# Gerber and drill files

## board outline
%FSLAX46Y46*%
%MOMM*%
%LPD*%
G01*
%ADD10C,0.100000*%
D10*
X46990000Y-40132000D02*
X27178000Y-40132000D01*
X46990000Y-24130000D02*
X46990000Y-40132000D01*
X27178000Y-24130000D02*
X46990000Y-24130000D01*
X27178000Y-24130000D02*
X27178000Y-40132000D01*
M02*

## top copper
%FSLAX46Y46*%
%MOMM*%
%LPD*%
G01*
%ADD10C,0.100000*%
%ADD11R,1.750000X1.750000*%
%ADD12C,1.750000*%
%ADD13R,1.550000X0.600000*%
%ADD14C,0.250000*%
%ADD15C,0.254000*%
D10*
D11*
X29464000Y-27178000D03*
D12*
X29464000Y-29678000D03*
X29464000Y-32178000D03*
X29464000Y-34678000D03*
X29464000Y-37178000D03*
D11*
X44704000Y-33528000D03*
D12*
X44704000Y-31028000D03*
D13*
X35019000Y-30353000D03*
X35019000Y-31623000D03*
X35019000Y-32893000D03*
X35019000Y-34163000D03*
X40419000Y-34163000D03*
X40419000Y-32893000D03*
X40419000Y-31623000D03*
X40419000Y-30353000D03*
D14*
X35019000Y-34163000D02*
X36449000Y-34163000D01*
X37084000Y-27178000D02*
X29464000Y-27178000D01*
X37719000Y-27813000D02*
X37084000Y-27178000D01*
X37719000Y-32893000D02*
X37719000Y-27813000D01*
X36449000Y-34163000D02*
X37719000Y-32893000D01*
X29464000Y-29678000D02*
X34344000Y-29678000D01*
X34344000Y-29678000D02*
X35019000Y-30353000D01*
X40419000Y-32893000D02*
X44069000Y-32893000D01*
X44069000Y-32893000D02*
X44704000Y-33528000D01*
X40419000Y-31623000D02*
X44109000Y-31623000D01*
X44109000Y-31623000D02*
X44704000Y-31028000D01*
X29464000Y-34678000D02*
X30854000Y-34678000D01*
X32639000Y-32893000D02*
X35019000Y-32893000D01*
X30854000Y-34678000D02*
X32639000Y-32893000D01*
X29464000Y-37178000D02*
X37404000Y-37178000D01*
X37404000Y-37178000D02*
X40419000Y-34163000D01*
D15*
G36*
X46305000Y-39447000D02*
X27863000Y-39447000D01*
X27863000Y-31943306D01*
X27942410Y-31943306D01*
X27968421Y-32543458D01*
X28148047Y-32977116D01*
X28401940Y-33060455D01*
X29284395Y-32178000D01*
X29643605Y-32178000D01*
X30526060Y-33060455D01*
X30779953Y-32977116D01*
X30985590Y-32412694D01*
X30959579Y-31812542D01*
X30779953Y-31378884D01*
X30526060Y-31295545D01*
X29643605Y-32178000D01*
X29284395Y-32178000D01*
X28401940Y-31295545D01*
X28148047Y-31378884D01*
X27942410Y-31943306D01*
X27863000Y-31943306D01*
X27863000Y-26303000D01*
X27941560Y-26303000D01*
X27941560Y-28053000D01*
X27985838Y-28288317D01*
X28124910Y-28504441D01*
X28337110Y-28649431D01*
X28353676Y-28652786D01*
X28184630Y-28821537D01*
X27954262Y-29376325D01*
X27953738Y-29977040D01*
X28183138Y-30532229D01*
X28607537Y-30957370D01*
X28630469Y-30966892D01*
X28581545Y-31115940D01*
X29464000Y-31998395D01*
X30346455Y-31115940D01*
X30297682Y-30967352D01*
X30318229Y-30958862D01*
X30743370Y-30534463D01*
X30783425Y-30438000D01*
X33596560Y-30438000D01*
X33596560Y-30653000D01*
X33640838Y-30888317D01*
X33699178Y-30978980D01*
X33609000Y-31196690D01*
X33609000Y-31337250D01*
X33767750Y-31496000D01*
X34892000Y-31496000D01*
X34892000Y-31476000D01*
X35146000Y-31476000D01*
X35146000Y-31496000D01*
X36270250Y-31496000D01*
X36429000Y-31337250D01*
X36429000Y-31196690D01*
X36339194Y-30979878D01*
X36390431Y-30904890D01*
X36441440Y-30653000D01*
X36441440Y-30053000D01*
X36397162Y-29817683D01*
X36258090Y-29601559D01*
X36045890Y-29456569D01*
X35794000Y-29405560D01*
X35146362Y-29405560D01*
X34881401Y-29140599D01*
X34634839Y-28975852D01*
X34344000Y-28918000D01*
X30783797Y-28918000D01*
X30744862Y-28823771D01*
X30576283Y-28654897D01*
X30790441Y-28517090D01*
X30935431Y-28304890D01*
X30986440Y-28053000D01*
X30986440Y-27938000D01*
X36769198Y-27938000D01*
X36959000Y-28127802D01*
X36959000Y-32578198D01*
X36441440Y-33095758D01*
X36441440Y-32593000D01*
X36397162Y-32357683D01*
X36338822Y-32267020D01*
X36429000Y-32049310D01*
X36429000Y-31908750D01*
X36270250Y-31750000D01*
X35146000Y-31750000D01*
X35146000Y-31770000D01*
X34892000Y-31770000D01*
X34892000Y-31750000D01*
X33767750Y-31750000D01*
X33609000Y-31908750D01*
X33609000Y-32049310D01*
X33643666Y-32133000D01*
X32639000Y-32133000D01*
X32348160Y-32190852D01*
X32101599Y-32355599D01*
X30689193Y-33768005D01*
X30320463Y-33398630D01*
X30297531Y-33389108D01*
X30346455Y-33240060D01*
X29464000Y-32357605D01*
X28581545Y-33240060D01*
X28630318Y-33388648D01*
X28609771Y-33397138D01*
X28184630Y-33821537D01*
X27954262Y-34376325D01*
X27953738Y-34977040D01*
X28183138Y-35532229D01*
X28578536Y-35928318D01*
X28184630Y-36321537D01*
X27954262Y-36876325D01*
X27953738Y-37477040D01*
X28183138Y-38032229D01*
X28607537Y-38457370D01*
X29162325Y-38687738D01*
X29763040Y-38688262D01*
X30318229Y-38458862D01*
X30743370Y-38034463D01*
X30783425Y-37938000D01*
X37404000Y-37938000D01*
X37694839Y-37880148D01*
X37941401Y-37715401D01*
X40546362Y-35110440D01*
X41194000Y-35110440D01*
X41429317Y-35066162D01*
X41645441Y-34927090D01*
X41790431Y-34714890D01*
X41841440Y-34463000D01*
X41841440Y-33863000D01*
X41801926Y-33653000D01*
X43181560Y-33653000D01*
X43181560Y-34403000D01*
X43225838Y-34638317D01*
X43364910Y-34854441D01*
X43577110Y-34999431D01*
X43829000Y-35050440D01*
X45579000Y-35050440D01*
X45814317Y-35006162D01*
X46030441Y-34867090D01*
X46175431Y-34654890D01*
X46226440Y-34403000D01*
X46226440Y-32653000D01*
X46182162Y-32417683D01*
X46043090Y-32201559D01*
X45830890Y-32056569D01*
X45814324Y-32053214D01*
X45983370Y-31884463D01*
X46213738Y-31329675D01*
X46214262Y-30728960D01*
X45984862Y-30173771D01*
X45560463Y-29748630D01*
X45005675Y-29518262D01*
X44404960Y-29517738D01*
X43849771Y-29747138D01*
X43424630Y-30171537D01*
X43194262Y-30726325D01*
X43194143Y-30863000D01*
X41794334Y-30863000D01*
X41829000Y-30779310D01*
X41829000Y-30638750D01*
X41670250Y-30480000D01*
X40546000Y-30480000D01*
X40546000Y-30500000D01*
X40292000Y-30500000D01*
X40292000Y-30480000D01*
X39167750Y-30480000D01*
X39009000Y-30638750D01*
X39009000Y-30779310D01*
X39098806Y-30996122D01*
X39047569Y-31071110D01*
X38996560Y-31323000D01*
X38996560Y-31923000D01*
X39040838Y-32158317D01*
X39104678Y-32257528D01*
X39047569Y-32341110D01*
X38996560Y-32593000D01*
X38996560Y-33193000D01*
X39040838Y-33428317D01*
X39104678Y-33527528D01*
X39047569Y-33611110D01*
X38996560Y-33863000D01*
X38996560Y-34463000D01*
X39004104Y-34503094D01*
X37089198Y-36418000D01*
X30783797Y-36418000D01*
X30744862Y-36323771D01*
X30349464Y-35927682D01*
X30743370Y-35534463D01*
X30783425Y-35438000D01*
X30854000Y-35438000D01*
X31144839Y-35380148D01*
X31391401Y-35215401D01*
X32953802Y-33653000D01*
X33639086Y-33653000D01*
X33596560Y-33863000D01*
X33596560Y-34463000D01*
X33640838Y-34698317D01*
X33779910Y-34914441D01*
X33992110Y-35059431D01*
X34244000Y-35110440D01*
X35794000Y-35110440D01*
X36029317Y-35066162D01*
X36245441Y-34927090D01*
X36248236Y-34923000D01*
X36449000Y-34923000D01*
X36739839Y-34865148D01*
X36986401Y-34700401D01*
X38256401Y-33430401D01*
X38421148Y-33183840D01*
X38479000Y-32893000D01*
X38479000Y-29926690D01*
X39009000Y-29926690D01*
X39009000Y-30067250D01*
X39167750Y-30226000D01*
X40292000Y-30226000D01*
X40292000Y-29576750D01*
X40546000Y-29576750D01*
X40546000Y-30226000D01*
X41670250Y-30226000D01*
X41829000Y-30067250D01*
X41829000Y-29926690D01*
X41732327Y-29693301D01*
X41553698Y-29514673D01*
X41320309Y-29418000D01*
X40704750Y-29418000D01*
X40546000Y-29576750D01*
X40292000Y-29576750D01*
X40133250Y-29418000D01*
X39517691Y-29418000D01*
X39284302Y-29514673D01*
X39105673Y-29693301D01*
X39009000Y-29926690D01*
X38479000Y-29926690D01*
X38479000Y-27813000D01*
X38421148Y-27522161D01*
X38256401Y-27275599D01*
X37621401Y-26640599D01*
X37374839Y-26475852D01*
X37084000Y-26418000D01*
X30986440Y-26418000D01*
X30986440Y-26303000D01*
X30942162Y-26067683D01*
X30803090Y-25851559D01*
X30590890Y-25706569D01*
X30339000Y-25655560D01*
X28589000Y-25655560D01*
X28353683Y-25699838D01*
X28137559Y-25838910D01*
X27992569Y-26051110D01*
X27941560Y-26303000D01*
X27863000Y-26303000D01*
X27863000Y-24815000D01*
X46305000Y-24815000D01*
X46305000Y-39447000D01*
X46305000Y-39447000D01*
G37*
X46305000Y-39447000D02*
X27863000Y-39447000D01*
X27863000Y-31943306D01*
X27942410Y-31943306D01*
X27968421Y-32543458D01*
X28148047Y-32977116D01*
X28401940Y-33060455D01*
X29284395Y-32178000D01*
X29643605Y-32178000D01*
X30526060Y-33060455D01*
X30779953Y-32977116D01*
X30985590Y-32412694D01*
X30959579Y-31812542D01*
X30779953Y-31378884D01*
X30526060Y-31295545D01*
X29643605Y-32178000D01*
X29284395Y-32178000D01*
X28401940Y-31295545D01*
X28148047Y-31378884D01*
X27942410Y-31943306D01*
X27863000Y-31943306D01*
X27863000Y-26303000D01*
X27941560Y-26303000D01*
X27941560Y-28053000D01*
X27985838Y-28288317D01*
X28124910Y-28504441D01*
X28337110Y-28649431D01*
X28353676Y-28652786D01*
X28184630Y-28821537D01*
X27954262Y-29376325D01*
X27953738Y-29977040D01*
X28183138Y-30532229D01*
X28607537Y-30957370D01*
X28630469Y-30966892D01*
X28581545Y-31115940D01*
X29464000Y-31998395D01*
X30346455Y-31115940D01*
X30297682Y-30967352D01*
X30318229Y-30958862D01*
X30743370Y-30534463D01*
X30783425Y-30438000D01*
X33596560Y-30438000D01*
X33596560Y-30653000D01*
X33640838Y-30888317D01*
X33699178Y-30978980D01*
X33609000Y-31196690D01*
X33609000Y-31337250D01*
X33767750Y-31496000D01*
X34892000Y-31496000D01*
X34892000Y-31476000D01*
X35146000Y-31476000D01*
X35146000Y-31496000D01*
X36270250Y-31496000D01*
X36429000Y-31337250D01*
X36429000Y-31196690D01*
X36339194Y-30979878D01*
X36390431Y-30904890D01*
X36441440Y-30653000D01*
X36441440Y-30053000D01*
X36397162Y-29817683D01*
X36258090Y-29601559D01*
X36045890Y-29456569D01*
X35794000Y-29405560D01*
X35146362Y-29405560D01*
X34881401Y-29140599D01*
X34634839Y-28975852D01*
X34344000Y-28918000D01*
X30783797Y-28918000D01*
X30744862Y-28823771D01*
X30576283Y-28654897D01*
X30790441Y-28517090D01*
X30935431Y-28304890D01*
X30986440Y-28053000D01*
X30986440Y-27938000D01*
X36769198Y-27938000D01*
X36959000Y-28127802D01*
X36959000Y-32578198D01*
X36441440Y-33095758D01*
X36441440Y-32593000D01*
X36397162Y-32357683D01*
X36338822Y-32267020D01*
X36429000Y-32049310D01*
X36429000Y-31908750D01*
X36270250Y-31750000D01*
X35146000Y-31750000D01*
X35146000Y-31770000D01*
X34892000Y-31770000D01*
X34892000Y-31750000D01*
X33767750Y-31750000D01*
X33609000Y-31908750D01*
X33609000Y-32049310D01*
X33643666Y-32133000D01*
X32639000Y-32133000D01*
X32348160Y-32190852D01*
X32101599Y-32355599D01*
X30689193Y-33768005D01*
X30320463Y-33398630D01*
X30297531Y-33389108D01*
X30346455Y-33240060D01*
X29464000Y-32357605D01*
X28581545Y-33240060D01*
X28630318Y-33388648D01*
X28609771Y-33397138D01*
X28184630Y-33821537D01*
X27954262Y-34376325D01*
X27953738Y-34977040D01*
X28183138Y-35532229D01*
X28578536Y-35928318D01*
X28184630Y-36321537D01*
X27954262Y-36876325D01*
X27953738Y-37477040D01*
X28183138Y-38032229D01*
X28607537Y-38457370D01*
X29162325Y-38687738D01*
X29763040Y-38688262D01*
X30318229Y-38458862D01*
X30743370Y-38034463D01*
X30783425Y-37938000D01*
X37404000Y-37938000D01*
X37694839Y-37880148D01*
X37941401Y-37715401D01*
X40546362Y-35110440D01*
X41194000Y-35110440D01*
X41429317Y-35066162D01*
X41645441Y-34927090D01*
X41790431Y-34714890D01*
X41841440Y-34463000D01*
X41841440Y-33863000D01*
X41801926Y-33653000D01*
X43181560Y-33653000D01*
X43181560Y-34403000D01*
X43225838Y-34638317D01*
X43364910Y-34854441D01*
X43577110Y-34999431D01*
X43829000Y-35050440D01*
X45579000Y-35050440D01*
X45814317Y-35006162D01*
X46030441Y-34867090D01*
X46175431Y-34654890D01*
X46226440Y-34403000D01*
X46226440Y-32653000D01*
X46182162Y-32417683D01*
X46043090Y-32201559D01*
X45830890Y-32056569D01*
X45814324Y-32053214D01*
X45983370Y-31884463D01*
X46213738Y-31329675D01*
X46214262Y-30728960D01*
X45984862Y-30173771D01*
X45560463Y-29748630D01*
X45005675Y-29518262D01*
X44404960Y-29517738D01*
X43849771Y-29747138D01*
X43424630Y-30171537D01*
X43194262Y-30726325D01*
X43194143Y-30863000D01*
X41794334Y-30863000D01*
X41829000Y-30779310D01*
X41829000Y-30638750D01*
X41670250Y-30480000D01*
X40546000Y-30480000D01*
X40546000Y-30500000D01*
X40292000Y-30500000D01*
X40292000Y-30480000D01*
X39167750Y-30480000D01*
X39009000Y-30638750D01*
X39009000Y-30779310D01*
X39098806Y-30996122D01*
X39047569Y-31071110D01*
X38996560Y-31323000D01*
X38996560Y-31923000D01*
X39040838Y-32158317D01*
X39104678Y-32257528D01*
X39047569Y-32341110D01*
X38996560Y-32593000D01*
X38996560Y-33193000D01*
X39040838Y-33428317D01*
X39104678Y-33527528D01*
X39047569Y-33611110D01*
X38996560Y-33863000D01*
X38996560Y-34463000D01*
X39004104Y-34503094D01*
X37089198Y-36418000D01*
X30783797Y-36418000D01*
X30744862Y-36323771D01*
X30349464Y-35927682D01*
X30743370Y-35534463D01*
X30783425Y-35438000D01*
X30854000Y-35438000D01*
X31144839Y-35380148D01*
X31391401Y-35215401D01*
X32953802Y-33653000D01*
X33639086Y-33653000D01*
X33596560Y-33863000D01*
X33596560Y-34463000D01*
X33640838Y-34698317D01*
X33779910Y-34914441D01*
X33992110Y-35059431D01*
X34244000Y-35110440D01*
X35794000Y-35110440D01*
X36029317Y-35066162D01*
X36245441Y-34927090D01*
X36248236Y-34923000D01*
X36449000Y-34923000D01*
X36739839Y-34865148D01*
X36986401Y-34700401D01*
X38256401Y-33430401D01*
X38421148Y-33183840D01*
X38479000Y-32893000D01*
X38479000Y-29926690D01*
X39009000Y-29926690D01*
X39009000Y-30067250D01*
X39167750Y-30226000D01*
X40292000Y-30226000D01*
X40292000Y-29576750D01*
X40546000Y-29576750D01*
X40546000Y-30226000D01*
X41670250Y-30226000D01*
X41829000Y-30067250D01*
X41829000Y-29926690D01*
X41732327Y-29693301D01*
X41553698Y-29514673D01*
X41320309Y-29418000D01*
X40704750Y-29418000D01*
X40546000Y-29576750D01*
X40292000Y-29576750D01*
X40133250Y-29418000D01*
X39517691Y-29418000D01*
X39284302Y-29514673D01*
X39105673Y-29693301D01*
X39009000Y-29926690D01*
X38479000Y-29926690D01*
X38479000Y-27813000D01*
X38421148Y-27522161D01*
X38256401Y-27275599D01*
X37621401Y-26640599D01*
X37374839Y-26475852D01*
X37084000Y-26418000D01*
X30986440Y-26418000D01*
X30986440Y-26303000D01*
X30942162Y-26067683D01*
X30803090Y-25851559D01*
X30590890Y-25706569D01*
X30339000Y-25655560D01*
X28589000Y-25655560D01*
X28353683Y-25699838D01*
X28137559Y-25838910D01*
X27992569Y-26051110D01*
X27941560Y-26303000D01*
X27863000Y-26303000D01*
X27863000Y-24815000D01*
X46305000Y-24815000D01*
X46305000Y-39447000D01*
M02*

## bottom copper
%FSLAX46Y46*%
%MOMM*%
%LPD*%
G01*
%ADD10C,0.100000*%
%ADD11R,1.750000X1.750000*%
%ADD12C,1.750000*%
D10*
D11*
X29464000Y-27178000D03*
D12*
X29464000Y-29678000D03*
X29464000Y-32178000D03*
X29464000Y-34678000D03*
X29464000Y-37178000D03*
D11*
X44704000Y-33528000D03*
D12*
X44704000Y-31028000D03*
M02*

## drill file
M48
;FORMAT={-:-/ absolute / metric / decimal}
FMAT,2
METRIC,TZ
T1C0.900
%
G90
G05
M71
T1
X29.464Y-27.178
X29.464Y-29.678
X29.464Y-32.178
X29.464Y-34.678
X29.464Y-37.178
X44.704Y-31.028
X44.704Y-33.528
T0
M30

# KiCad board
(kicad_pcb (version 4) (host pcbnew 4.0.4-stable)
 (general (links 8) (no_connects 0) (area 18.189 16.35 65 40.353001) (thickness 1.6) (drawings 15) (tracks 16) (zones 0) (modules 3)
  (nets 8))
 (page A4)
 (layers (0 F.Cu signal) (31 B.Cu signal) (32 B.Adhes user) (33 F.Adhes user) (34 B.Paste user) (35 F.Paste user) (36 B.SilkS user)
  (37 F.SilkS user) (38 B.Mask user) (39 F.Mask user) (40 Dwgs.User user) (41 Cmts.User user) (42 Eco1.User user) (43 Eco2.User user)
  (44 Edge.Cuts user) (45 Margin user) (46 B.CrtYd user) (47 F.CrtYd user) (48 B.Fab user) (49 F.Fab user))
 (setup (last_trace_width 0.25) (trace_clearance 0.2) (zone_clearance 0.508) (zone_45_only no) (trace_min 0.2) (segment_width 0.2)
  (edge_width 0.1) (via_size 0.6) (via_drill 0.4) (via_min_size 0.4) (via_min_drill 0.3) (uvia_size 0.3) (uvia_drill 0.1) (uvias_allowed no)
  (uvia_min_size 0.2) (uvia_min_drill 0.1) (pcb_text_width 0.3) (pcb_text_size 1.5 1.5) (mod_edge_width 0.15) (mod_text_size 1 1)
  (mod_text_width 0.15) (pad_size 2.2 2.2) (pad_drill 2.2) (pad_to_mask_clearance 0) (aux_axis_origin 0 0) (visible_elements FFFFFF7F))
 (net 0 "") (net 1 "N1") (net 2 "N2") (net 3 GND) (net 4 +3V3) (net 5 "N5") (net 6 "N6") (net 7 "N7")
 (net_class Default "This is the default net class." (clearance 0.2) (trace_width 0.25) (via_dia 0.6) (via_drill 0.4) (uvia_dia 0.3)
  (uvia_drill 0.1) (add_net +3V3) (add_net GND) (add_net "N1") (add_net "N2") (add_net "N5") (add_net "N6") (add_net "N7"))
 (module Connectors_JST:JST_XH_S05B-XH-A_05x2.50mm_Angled (layer F.Cu) (at 29.464 27.178 270)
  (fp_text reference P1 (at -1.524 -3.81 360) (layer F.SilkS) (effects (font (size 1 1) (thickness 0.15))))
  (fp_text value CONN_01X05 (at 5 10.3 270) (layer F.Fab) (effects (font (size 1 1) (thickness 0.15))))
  (pad 1 thru_hole rect (at 0 0 270) (size 1.75 1.75) (drill 0.9) (layers *.Cu *.Mask F.SilkS) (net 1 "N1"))
  (pad 2 thru_hole circle (at 2.5 0 270) (size 1.75 1.75) (drill 0.9) (layers *.Cu *.Mask F.SilkS) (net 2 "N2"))
  (pad 3 thru_hole circle (at 5 0 270) (size 1.75 1.75) (drill 0.9) (layers *.Cu *.Mask F.SilkS) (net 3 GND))
  (pad 4 thru_hole circle (at 7.5 0 270) (size 1.75 1.75) (drill 0.9) (layers *.Cu *.Mask F.SilkS) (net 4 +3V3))
  (pad 5 thru_hole circle (at 10 0 270) (size 1.75 1.75) (drill 0.9) (layers *.Cu *.Mask F.SilkS) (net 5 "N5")))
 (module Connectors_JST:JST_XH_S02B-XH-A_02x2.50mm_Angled (layer F.Cu) (at 44.704 33.528 90)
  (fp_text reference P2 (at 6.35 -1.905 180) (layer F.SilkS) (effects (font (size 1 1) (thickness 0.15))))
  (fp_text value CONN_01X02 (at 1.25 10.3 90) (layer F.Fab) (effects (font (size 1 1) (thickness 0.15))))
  (pad 1 thru_hole rect (at 0 0 90) (size 1.75 1.75) (drill 0.9) (layers *.Cu *.Mask F.SilkS) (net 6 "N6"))
  (pad 2 thru_hole circle (at 2.5 0 90) (size 1.75 1.75) (drill 0.9) (layers *.Cu *.Mask F.SilkS) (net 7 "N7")))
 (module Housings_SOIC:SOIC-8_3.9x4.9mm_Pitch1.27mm (layer F.Cu) (at 37.719 32.258)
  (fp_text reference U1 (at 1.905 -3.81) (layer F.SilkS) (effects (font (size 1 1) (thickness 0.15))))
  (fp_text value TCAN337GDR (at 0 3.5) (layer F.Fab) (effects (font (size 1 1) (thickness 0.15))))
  (pad 1 smd rect (at -2.7 -1.905) (size 1.55 0.6) (layers F.Cu F.Paste F.Mask) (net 2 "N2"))
  (pad 2 smd rect (at -2.7 -0.635) (size 1.55 0.6) (layers F.Cu F.Paste F.Mask) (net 3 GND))
  (pad 3 smd rect (at -2.7 0.635) (size 1.55 0.6) (layers F.Cu F.Paste F.Mask) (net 4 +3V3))
  (pad 4 smd rect (at -2.7 1.905) (size 1.55 0.6) (layers F.Cu F.Paste F.Mask) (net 1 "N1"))
  (pad 5 smd rect (at 2.7 1.905) (size 1.55 0.6) (layers F.Cu F.Paste F.Mask) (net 5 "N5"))
  (pad 6 smd rect (at 2.7 0.635) (size 1.55 0.6) (layers F.Cu F.Paste F.Mask) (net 6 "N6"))
  (pad 7 smd rect (at 2.7 -0.635) (size 1.55 0.6) (layers F.Cu F.Paste F.Mask) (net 7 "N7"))
  (pad 8 smd rect (at 2.7 -1.905) (size 1.55 0.6) (layers F.Cu F.Paste F.Mask) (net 3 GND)))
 (gr_line (start 46.99 40.132) (end 27.178 40.132) (angle 90) (layer Edge.Cuts) (width 0.1))
 (gr_line (start 46.99 24.13) (end 46.99 40.132) (angle 90) (layer Edge.Cuts) (width 0.1))
 (gr_line (start 27.178 24.13) (end 46.99 24.13) (angle 90) (layer Edge.Cuts) (width 0.1))
 (gr_line (start 27.178 24.13) (end 27.178 40.132) (angle 90) (layer Edge.Cuts) (width 0.1))
 (segment (start 35.019 34.163) (end 36.449 34.163) (width 0.25) (layer F.Cu) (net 1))
 (segment (start 37.084 27.178) (end 29.464 27.178) (width 0.25) (layer F.Cu) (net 1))
 (segment (start 37.719 27.813) (end 37.084 27.178) (width 0.25) (layer F.Cu) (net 1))
 (segment (start 37.719 32.893) (end 37.719 27.813) (width 0.25) (layer F.Cu) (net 1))
 (segment (start 36.449 34.163) (end 37.719 32.893) (width 0.25) (layer F.Cu) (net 1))
 (segment (start 29.464 29.678) (end 34.344 29.678) (width 0.25) (layer F.Cu) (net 2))
 (segment (start 34.344 29.678) (end 35.019 30.353) (width 0.25) (layer F.Cu) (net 2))
 (segment (start 40.419 32.893) (end 44.069 32.893) (width 0.25) (layer F.Cu) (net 6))
 (segment (start 44.069 32.893) (end 44.704 33.528) (width 0.25) (layer F.Cu) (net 6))
 (segment (start 40.419 31.623) (end 44.109 31.623) (width 0.25) (layer F.Cu) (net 7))
 (segment (start 44.109 31.623) (end 44.704 31.028) (width 0.25) (layer F.Cu) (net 7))
 (segment (start 29.464 34.678) (end 30.854 34.678) (width 0.25) (layer F.Cu) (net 4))
 (segment (start 32.639 32.893) (end 35.019 32.893) (width 0.25) (layer F.Cu) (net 4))
 (segment (start 30.854 34.678) (end 32.639 32.893) (width 0.25) (layer F.Cu) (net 4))
 (segment (start 29.464 37.178) (end 37.404 37.178) (width 0.25) (layer F.Cu) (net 5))
 (segment (start 37.404 37.178) (end 40.419 34.163) (width 0.25) (layer F.Cu) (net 5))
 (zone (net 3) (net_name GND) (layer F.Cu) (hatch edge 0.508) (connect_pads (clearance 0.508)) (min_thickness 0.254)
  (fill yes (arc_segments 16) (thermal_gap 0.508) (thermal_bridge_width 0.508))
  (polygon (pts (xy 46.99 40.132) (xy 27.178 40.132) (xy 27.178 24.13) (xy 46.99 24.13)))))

